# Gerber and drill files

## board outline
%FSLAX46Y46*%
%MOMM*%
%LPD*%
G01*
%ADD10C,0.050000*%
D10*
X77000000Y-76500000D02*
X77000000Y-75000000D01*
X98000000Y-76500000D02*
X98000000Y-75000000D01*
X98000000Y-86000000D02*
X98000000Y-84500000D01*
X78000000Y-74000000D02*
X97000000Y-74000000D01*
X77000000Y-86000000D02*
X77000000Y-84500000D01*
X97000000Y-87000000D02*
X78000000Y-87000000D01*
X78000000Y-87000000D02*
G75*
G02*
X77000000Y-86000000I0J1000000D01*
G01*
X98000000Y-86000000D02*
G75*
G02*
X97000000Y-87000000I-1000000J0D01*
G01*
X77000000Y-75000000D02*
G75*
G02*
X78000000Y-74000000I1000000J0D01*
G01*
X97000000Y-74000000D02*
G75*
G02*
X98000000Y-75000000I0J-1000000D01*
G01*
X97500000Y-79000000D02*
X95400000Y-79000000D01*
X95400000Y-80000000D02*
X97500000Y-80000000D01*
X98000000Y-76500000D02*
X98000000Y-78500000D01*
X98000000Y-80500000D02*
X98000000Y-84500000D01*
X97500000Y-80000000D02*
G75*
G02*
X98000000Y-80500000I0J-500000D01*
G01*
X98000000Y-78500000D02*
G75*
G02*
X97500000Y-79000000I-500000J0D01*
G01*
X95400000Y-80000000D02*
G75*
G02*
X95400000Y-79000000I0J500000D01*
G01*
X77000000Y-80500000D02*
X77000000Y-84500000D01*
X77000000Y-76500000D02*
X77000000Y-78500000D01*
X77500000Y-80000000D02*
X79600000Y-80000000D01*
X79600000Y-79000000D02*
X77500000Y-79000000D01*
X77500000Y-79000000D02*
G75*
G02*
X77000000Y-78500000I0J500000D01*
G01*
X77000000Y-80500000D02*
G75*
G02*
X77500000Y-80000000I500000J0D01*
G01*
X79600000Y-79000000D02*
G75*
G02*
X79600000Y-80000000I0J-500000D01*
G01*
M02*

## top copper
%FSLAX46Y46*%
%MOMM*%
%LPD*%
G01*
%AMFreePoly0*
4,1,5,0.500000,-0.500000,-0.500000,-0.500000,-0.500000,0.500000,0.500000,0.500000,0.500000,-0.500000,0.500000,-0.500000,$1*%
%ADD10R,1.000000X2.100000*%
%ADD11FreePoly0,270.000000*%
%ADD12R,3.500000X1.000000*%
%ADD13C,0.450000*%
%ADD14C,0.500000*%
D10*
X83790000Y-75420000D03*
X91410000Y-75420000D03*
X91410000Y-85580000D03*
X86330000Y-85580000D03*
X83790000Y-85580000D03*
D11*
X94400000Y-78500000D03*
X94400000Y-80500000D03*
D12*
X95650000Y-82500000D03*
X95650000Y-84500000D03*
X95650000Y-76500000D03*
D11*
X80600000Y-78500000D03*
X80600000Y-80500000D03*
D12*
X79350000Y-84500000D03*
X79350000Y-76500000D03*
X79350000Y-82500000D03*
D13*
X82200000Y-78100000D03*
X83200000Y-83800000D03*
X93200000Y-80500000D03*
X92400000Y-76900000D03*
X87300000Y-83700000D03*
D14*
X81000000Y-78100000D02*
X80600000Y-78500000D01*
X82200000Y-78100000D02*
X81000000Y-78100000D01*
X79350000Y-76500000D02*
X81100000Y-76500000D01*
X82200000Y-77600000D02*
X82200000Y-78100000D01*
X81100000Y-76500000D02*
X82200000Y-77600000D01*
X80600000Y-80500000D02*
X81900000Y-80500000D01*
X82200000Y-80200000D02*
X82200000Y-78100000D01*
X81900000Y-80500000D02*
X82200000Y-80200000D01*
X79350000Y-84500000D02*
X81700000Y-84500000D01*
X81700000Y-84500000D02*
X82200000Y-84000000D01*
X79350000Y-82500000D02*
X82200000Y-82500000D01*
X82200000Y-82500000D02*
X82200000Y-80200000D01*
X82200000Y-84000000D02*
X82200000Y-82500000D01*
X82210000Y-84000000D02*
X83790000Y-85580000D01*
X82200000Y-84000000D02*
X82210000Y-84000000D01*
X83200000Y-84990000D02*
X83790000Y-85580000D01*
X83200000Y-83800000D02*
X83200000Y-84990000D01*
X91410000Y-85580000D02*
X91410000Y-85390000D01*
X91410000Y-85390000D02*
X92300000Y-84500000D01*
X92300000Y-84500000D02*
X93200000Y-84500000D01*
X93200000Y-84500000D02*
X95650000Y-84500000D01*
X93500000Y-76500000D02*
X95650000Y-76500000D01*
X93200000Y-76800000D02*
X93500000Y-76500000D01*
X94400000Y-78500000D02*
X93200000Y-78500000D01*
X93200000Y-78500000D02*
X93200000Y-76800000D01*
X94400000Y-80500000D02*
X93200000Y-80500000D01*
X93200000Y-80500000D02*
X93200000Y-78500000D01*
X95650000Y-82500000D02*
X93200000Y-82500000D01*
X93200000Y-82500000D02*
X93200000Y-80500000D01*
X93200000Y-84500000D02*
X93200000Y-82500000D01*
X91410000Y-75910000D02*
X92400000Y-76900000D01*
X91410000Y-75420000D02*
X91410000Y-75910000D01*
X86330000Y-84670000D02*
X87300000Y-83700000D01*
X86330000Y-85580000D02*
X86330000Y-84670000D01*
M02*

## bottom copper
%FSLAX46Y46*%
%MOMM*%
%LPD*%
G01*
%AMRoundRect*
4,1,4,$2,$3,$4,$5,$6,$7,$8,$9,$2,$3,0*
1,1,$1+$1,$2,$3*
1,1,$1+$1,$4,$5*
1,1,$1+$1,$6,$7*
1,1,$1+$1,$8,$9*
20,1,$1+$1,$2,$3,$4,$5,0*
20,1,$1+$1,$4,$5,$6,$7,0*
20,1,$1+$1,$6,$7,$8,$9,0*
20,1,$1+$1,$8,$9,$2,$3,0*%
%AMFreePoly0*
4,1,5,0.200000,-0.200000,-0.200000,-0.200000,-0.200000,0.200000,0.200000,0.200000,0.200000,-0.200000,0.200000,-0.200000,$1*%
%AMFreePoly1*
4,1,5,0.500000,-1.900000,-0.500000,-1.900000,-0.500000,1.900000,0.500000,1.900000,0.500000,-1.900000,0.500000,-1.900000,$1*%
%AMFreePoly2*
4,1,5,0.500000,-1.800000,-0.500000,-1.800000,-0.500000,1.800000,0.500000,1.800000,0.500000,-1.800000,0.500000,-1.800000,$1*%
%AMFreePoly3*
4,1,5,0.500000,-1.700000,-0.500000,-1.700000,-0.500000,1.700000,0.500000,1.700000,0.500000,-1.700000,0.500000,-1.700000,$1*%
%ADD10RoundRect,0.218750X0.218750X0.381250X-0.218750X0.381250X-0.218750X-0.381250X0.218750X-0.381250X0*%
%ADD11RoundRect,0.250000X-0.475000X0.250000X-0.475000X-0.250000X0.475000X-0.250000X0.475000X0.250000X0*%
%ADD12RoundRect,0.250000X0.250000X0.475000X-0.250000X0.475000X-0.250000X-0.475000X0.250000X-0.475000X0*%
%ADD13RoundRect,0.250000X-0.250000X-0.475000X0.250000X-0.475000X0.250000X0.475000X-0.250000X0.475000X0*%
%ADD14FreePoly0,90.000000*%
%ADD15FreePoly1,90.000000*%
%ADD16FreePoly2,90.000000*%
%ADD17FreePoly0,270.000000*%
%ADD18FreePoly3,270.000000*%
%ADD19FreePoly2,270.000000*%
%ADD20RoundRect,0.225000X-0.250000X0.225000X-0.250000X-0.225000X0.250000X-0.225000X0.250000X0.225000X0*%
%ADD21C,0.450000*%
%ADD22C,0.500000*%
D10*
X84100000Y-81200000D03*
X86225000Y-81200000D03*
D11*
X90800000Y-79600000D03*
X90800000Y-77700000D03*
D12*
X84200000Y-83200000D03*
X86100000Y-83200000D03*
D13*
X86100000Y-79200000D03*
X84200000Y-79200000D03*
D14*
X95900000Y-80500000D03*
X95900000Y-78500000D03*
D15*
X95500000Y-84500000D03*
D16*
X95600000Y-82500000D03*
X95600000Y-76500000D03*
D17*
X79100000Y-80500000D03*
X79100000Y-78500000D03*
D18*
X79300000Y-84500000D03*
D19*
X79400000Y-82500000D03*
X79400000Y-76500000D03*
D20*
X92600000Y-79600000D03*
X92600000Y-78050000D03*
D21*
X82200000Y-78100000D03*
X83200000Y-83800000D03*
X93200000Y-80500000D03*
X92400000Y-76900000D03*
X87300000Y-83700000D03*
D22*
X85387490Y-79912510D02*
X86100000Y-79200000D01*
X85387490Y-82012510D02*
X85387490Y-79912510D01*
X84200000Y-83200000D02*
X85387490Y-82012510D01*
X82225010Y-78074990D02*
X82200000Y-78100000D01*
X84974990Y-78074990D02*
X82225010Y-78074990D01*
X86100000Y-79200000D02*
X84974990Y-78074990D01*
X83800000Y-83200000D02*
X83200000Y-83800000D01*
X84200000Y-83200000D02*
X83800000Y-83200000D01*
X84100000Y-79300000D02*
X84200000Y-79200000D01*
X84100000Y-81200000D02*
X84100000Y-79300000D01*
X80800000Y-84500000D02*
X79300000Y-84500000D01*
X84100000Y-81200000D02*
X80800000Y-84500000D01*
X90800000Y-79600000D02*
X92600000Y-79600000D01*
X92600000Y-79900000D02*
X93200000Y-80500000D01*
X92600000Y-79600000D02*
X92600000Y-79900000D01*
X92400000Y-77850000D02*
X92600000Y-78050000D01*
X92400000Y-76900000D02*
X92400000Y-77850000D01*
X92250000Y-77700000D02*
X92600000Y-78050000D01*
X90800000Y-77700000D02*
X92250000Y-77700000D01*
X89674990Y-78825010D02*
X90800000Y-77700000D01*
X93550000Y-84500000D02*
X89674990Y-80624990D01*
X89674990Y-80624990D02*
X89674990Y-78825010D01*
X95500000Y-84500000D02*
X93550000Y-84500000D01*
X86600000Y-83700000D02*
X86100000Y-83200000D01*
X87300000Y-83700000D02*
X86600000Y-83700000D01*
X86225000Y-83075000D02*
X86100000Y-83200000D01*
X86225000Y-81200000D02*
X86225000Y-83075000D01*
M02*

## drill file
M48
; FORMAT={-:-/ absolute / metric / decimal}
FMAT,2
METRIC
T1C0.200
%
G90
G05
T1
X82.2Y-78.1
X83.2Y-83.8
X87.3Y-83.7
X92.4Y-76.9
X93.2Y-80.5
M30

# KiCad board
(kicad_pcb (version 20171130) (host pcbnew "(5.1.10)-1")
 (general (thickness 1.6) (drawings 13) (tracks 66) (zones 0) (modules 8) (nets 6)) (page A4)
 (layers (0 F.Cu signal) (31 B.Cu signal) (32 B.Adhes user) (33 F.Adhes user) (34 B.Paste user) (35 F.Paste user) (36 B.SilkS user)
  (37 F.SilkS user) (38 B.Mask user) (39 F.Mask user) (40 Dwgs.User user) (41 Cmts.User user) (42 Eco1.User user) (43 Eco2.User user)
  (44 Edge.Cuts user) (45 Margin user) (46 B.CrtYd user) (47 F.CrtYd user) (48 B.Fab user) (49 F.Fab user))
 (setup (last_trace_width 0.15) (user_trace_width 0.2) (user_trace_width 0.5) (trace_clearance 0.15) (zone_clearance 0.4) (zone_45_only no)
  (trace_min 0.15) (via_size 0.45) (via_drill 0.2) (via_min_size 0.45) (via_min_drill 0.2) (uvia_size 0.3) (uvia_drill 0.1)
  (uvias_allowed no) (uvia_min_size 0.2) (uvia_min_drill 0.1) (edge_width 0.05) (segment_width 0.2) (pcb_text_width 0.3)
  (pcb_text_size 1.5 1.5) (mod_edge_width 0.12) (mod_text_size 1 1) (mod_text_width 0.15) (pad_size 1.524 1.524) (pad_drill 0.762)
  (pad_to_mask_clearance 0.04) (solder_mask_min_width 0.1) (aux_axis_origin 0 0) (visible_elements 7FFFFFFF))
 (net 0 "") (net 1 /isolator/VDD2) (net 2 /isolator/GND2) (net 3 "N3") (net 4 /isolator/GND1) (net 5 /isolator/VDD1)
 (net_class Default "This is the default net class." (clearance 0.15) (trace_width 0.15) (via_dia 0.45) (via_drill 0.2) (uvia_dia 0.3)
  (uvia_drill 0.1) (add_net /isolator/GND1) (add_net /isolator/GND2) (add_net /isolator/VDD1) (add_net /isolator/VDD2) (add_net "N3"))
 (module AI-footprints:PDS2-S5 (layer F.Cu) (at 87.6 80.5)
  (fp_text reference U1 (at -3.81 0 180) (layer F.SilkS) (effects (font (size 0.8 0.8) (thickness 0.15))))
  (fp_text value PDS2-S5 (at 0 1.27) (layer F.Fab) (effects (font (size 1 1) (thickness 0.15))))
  (pad 8 smd rect (at -3.81 -5.08) (size 1 2.1) (layers F.Cu F.Paste F.Mask))
  (pad 5 smd rect (at 3.81 -5.08) (size 1 2.1) (layers F.Cu F.Paste F.Mask) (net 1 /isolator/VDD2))
  (pad 4 smd rect (at 3.81 5.08) (size 1 2.1) (layers F.Cu F.Paste F.Mask) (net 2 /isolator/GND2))
  (pad 2 smd rect (at -1.27 5.08) (size 1 2.1) (layers F.Cu F.Paste F.Mask) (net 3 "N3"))
  (pad 1 smd rect (at -3.81 5.08) (size 1 2.1) (layers F.Cu F.Paste F.Mask) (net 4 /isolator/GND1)))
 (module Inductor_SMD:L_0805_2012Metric (layer B.Cu) (at 85.1625 81.2 180)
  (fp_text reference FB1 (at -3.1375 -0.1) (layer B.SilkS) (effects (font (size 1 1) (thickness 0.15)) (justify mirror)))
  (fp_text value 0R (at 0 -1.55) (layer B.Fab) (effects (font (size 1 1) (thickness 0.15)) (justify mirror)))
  (pad 2 smd roundrect (at 1.0625 0 180) (size 0.875 1.2) (layers B.Cu B.Paste B.Mask) (roundrect_rratio 0.25) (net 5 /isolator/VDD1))
  (pad 1 smd roundrect (at -1.0625 0 180) (size 0.875 1.2) (layers B.Cu B.Paste B.Mask) (roundrect_rratio 0.25) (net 3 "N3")))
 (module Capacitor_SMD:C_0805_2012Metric (layer B.Cu) (at 90.8 78.65 270)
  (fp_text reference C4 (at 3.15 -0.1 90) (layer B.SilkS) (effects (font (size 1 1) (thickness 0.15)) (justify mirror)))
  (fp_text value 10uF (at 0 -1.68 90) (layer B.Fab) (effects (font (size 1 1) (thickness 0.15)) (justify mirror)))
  (pad 2 smd roundrect (at 0.95 0 270) (size 1 1.45) (layers B.Cu B.Paste B.Mask) (roundrect_rratio 0.25) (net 2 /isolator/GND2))
  (pad 1 smd roundrect (at -0.95 0 270) (size 1 1.45) (layers B.Cu B.Paste B.Mask) (roundrect_rratio 0.25) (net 1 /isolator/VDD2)))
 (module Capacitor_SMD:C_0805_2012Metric (layer B.Cu) (at 85.15 83.2 180)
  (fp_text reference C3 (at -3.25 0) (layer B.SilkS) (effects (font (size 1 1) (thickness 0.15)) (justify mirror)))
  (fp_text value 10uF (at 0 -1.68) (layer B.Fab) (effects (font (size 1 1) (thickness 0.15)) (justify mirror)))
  (pad 2 smd roundrect (at 0.95 0 180) (size 1 1.45) (layers B.Cu B.Paste B.Mask) (roundrect_rratio 0.25) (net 4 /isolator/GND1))
  (pad 1 smd roundrect (at -0.95 0 180) (size 1 1.45) (layers B.Cu B.Paste B.Mask) (roundrect_rratio 0.25) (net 3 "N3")))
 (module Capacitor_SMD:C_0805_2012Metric (layer B.Cu) (at 85.15 79.2)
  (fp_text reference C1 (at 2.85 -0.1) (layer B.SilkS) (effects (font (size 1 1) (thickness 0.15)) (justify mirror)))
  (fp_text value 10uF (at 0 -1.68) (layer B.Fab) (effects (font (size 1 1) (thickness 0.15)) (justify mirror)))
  (pad 2 smd roundrect (at 0.95 0) (size 1 1.45) (layers B.Cu B.Paste B.Mask) (roundrect_rratio 0.25) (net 4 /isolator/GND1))
  (pad 1 smd roundrect (at -0.95 0) (size 1 1.45) (layers B.Cu B.Paste B.Mask) (roundrect_rratio 0.25) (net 5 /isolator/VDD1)))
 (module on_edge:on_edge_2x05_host (layer F.Cu) (at 98 80.5 270)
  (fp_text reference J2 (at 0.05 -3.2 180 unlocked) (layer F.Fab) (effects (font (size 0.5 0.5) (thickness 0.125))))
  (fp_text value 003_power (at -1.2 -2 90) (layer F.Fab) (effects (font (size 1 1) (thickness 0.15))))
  (fp_line (start -1.5 0.5) (end -1.5 2.6) (layer Edge.Cuts) (width 0.05))
  (fp_line (start -0.5 2.6) (end -0.5 0.5) (layer Edge.Cuts) (width 0.05))
  (fp_line (start -4 0) (end -2 0) (layer Edge.Cuts) (width 0.05))
  (fp_line (start 0 0) (end 4 0) (layer Edge.Cuts) (width 0.05))
  (fp_arc (start 0 0.5) (end 0 0) (angle -90) (layer Edge.Cuts) (width 0.05))
  (fp_arc (start -2 0.5) (end -1.5 0.5) (angle -90) (layer Edge.Cuts) (width 0.05))
  (fp_arc (start -1 2.6) (end -1.5 2.6) (angle -180) (layer Edge.Cuts) (width 0.05))
  (pad 2 smd custom (at -2 3.6 270) (size 1 1) (layers F.Cu F.Mask) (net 2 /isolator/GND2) (zone_connect 0)
   (options (clearance outline) (anchor rect)) (primitives))
  (pad 3 smd custom (at 0 3.6 270) (size 1 1) (layers F.Cu F.Mask) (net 2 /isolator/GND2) (zone_connect 0)
   (options (clearance outline) (anchor rect)) (primitives))
  (pad 8 smd custom (at 0 2.1 90) (size 0.4 0.4) (layers B.Cu B.Mask) (zone_connect 0) (options (clearance outline) (anchor rect))
   (primitives))
  (pad 7 smd custom (at -2 2.1 90) (size 0.4 0.4) (layers B.Cu B.Mask) (zone_connect 0) (options (clearance outline) (anchor rect))
   (primitives))
  (pad 4 smd rect (at 2 2.35 270) (size 1 3.5) (layers F.Cu F.Mask) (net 2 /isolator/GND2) (zone_connect 0))
  (pad 10 smd custom (at 4 2.5 90) (size 1 3.8) (layers B.Cu B.Mask) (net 1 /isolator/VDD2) (zone_connect 0)
   (options (clearance outline) (anchor rect)) (primitives))
  (pad 9 smd custom (at 2 2.4 90) (size 1 3.6) (layers B.Cu B.Mask) (zone_connect 0) (options (clearance outline) (anchor rect))
   (primitives))
  (pad 6 smd custom (at -4 2.4 90) (size 1 3.6) (layers B.Cu B.Mask) (zone_connect 0) (options (clearance outline) (anchor rect))
   (primitives))
  (pad 5 smd rect (at 4 2.35 270) (size 1 3.5) (layers F.Cu F.Mask) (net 2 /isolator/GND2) (zone_connect 0))
  (pad 1 smd rect (at -4 2.35 270) (size 1 3.5) (layers F.Cu F.Mask) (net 2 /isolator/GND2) (zone_connect 0)))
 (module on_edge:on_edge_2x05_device (layer F.Cu) (at 77 80.5 270)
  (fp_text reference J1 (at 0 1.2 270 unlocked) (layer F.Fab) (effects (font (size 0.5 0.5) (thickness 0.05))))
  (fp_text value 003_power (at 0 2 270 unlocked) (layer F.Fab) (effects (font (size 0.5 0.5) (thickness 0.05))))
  (fp_line (start 0 0) (end 4 0) (layer Edge.Cuts) (width 0.05))
  (fp_line (start -4 0) (end -2 0) (layer Edge.Cuts) (width 0.05))
  (fp_line (start -0.5 -0.5) (end -0.5 -2.6) (layer Edge.Cuts) (width 0.05))
  (fp_line (start -1.5 -2.6) (end -1.5 -0.5) (layer Edge.Cuts) (width 0.05))
  (fp_arc (start -2 -0.5) (end -2 0) (angle -90) (layer Edge.Cuts) (width 0.05))
  (fp_arc (start 0 -0.5) (end -0.5 -0.5) (angle -90) (layer Edge.Cuts) (width 0.05))
  (fp_arc (start -1 -2.6) (end -0.5 -2.6) (angle -180) (layer Edge.Cuts) (width 0.05))
  (pad 2 smd custom (at -2 -3.6 270) (size 1 1) (layers F.Cu F.Mask) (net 4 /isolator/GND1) (zone_connect 0)
   (options (clearance outline) (anchor rect)) (primitives))
  (pad 3 smd custom (at 0 -3.6 270) (size 1 1) (layers F.Cu F.Mask) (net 4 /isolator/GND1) (zone_connect 0)
   (options (clearance outline) (anchor rect)) (primitives))
  (pad 8 smd custom (at 0 -2.1 270) (size 0.4 0.4) (layers B.Cu B.Mask) (zone_connect 0) (options (clearance outline) (anchor rect))
   (primitives))
  (pad 7 smd custom (at -2 -2.1 270) (size 0.4 0.4) (layers B.Cu B.Mask) (zone_connect 0) (options (clearance outline) (anchor rect))
   (primitives))
  (pad 10 smd custom (at 4 -2.3 270) (size 1 3.4) (layers B.Cu B.Mask) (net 5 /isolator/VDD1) (zone_connect 0)
   (options (clearance outline) (anchor rect)) (primitives))
  (pad 9 smd custom (at 2 -2.4 270) (size 1 3.6) (layers B.Cu B.Mask) (zone_connect 0) (options (clearance outline) (anchor rect))
   (primitives))
  (pad 6 smd custom (at -4 -2.4 270) (size 1 3.6) (layers B.Cu B.Mask) (zone_connect 0) (options (clearance outline) (anchor rect))
   (primitives))
  (pad 5 smd rect (at 4 -2.35 90) (size 1 3.5) (layers F.Cu F.Mask) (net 4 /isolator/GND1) (zone_connect 0))
  (pad 1 smd rect (at -4 -2.35 90) (size 1 3.5) (layers F.Cu F.Mask) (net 4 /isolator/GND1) (zone_connect 0))
  (pad 4 smd rect (at 2 -2.35 90) (size 1 3.5) (layers F.Cu F.Mask) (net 4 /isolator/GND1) (zone_connect 0)))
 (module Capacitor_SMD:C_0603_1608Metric (layer B.Cu) (at 92.6 78.825 270)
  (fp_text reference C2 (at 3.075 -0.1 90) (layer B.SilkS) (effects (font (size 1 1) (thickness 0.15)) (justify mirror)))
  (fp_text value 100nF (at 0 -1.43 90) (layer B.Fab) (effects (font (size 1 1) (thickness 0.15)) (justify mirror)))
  (pad 2 smd roundrect (at 0.775 0 270) (size 0.9 0.95) (layers B.Cu B.Paste B.Mask) (roundrect_rratio 0.25) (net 2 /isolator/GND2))
  (pad 1 smd roundrect (at -0.775 0 270) (size 0.9 0.95) (layers B.Cu B.Paste B.Mask) (roundrect_rratio 0.25) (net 1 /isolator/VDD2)))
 (gr_line (start 77 76.5) (end 77 75) (layer Edge.Cuts) (width 0.05))
 (gr_line (start 98 76.5) (end 98 75) (layer Edge.Cuts) (width 0.05))
 (gr_line (start 98 86) (end 98 84.5) (layer Edge.Cuts) (width 0.05))
 (gr_line (start 78 74) (end 97 74) (layer Edge.Cuts) (width 0.05))
 (gr_line (start 77 86) (end 77 84.5) (layer Edge.Cuts) (width 0.05))
 (gr_line (start 97 87) (end 78 87) (layer Edge.Cuts) (width 0.05))
 (gr_arc (start 78 86) (end 77 86) (angle -90) (layer Edge.Cuts) (width 0.05))
 (gr_arc (start 97 86) (end 97 87) (angle -90) (layer Edge.Cuts) (width 0.05))
 (gr_arc (start 78 75) (end 78 74) (angle -90) (layer Edge.Cuts) (width 0.05))
 (gr_arc (start 97 75) (end 98 75) (angle -90) (layer Edge.Cuts) (width 0.05))
 (segment (start 85.38749 79.91251) (end 86.1 79.2) (width 0.5) (layer B.Cu) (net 4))
 (segment (start 85.38749 82.01251) (end 85.38749 79.91251) (width 0.5) (layer B.Cu) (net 4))
 (segment (start 84.2 83.2) (end 85.38749 82.01251) (width 0.5) (layer B.Cu) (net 4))
 (via (at 82.2 78.1) (size 0.45) (drill 0.2) (layers F.Cu B.Cu) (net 4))
 (segment (start 82.22501 78.07499) (end 82.2 78.1) (width 0.5) (layer B.Cu) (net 4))
 (segment (start 84.97499 78.07499) (end 82.22501 78.07499) (width 0.5) (layer B.Cu) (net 4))
 (segment (start 86.1 79.2) (end 84.97499 78.07499) (width 0.5) (layer B.Cu) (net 4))
 (segment (start 81 78.1) (end 80.6 78.5) (width 0.5) (layer F.Cu) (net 4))
 (segment (start 82.2 78.1) (end 81 78.1) (width 0.5) (layer F.Cu) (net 4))
 (segment (start 79.35 76.5) (end 81.1 76.5) (width 0.5) (layer F.Cu) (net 4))
 (segment (start 82.2 77.6) (end 82.2 78.1) (width 0.5) (layer F.Cu) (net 4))
 (segment (start 81.1 76.5) (end 82.2 77.6) (width 0.5) (layer F.Cu) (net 4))
 (segment (start 80.6 80.5) (end 81.9 80.5) (width 0.5) (layer F.Cu) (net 4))
 (segment (start 82.2 80.2) (end 82.2 78.1) (width 0.5) (layer F.Cu) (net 4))
 (segment (start 81.9 80.5) (end 82.2 80.2) (width 0.5) (layer F.Cu) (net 4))
 (segment (start 79.35 84.5) (end 81.7 84.5) (width 0.5) (layer F.Cu) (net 4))
 (segment (start 81.7 84.5) (end 82.2 84) (width 0.5) (layer F.Cu) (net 4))
 (segment (start 79.35 82.5) (end 82.2 82.5) (width 0.5) (layer F.Cu) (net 4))
 (segment (start 82.2 82.5) (end 82.2 80.2) (width 0.5) (layer F.Cu) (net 4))
 (segment (start 82.2 84) (end 82.2 82.5) (width 0.5) (layer F.Cu) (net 4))
 (segment (start 82.21 84) (end 83.79 85.58) (width 0.5) (layer F.Cu) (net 4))
 (segment (start 82.2 84) (end 82.21 84) (width 0.5) (layer F.Cu) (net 4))
 (via (at 83.2 83.8) (size 0.45) (drill 0.2) (layers F.Cu B.Cu) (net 4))
 (segment (start 83.8 83.2) (end 83.2 83.8) (width 0.5) (layer B.Cu) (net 4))
 (segment (start 84.2 83.2) (end 83.8 83.2) (width 0.5) (layer B.Cu) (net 4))
 (segment (start 83.2 84.99) (end 83.79 85.58) (width 0.5) (layer F.Cu) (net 4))
 (segment (start 83.2 83.8) (end 83.2 84.99) (width 0.5) (layer F.Cu) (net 4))
 (segment (start 84.1 79.3) (end 84.2 79.2) (width 0.5) (layer B.Cu) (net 5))
 (segment (start 84.1 81.2) (end 84.1 79.3) (width 0.5) (layer B.Cu) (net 5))
 (segment (start 80.8 84.5) (end 79.3 84.5) (width 0.5) (layer B.Cu) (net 5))
 (segment (start 84.1 81.2) (end 80.8 84.5) (width 0.5) (layer B.Cu) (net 5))
 (segment (start 90.8 79.6) (end 92.6 79.6) (width 0.5) (layer B.Cu) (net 2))
 (segment (start 91.41 85.58) (end 91.41 85.39) (width 0.5) (layer F.Cu) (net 2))
 (segment (start 91.41 85.39) (end 92.3 84.5) (width 0.5) (layer F.Cu) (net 2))
 (segment (start 92.3 84.5) (end 93.2 84.5) (width 0.5) (layer F.Cu) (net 2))
 (segment (start 93.2 84.5) (end 95.65 84.5) (width 0.5) (layer F.Cu) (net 2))
 (segment (start 93.5 76.5) (end 95.65 76.5) (width 0.5) (layer F.Cu) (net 2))
 (segment (start 93.2 76.8) (end 93.5 76.5) (width 0.5) (layer F.Cu) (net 2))
 (segment (start 94.4 78.5) (end 93.2 78.5) (width 0.5) (layer F.Cu) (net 2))
 (segment (start 93.2 78.5) (end 93.2 76.8) (width 0.5) (layer F.Cu) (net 2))
 (segment (start 94.4 80.5) (end 93.2 80.5) (width 0.5) (layer F.Cu) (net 2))
 (segment (start 93.2 80.5) (end 93.2 78.5) (width 0.5) (layer F.Cu) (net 2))
 (segment (start 95.65 82.5) (end 93.2 82.5) (width 0.5) (layer F.Cu) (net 2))
 (segment (start 93.2 82.5) (end 93.2 80.5) (width 0.5) (layer F.Cu) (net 2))
 (segment (start 93.2 84.5) (end 93.2 82.5) (width 0.5) (layer F.Cu) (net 2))
 (via (at 93.2 80.5) (size 0.45) (drill 0.2) (layers F.Cu B.Cu) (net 2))
 (segment (start 92.6 79.9) (end 93.2 80.5) (width 0.5) (layer B.Cu) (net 2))
 (segment (start 92.6 79.6) (end 92.6 79.9) (width 0.5) (layer B.Cu) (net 2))
 (via (at 92.4 76.9) (size 0.45) (drill 0.2) (layers F.Cu B.Cu) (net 1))
 (segment (start 91.41 75.91) (end 92.4 76.9) (width 0.5) (layer F.Cu) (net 1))
 (segment (start 91.41 75.42) (end 91.41 75.91) (width 0.5) (layer F.Cu) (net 1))
 (segment (start 92.4 77.85) (end 92.6 78.05) (width 0.5) (layer B.Cu) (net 1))
 (segment (start 92.4 76.9) (end 92.4 77.85) (width 0.5) (layer B.Cu) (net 1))
 (segment (start 92.25 77.7) (end 92.6 78.05) (width 0.5) (layer B.Cu) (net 1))
 (segment (start 90.8 77.7) (end 92.25 77.7) (width 0.5) (layer B.Cu) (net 1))
 (segment (start 89.67499 78.82501) (end 90.8 77.7) (width 0.5) (layer B.Cu) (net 1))
 (segment (start 93.55 84.5) (end 89.67499 80.62499) (width 0.5) (layer B.Cu) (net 1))
 (segment (start 89.67499 80.62499) (end 89.67499 78.82501) (width 0.5) (layer B.Cu) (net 1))
 (segment (start 95.5 84.5) (end 93.55 84.5) (width 0.5) (layer B.Cu) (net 1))
 (via (at 87.3 83.7) (size 0.45) (drill 0.2) (layers F.Cu B.Cu) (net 3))
 (segment (start 86.33 84.67) (end 87.3 83.7) (width 0.5) (layer F.Cu) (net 3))
 (segment (start 86.33 85.58) (end 86.33 84.67) (width 0.5) (layer F.Cu) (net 3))
 (segment (start 86.6 83.7) (end 86.1 83.2) (width 0.5) (layer B.Cu) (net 3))
 (segment (start 87.3 83.7) (end 86.6 83.7) (width 0.5) (layer B.Cu) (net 3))
 (segment (start 86.225 83.075) (end 86.1 83.2) (width 0.5) (layer B.Cu) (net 3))
 (segment (start 86.225 81.2) (end 86.225 83.075) (width 0.5) (layer B.Cu) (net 3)))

